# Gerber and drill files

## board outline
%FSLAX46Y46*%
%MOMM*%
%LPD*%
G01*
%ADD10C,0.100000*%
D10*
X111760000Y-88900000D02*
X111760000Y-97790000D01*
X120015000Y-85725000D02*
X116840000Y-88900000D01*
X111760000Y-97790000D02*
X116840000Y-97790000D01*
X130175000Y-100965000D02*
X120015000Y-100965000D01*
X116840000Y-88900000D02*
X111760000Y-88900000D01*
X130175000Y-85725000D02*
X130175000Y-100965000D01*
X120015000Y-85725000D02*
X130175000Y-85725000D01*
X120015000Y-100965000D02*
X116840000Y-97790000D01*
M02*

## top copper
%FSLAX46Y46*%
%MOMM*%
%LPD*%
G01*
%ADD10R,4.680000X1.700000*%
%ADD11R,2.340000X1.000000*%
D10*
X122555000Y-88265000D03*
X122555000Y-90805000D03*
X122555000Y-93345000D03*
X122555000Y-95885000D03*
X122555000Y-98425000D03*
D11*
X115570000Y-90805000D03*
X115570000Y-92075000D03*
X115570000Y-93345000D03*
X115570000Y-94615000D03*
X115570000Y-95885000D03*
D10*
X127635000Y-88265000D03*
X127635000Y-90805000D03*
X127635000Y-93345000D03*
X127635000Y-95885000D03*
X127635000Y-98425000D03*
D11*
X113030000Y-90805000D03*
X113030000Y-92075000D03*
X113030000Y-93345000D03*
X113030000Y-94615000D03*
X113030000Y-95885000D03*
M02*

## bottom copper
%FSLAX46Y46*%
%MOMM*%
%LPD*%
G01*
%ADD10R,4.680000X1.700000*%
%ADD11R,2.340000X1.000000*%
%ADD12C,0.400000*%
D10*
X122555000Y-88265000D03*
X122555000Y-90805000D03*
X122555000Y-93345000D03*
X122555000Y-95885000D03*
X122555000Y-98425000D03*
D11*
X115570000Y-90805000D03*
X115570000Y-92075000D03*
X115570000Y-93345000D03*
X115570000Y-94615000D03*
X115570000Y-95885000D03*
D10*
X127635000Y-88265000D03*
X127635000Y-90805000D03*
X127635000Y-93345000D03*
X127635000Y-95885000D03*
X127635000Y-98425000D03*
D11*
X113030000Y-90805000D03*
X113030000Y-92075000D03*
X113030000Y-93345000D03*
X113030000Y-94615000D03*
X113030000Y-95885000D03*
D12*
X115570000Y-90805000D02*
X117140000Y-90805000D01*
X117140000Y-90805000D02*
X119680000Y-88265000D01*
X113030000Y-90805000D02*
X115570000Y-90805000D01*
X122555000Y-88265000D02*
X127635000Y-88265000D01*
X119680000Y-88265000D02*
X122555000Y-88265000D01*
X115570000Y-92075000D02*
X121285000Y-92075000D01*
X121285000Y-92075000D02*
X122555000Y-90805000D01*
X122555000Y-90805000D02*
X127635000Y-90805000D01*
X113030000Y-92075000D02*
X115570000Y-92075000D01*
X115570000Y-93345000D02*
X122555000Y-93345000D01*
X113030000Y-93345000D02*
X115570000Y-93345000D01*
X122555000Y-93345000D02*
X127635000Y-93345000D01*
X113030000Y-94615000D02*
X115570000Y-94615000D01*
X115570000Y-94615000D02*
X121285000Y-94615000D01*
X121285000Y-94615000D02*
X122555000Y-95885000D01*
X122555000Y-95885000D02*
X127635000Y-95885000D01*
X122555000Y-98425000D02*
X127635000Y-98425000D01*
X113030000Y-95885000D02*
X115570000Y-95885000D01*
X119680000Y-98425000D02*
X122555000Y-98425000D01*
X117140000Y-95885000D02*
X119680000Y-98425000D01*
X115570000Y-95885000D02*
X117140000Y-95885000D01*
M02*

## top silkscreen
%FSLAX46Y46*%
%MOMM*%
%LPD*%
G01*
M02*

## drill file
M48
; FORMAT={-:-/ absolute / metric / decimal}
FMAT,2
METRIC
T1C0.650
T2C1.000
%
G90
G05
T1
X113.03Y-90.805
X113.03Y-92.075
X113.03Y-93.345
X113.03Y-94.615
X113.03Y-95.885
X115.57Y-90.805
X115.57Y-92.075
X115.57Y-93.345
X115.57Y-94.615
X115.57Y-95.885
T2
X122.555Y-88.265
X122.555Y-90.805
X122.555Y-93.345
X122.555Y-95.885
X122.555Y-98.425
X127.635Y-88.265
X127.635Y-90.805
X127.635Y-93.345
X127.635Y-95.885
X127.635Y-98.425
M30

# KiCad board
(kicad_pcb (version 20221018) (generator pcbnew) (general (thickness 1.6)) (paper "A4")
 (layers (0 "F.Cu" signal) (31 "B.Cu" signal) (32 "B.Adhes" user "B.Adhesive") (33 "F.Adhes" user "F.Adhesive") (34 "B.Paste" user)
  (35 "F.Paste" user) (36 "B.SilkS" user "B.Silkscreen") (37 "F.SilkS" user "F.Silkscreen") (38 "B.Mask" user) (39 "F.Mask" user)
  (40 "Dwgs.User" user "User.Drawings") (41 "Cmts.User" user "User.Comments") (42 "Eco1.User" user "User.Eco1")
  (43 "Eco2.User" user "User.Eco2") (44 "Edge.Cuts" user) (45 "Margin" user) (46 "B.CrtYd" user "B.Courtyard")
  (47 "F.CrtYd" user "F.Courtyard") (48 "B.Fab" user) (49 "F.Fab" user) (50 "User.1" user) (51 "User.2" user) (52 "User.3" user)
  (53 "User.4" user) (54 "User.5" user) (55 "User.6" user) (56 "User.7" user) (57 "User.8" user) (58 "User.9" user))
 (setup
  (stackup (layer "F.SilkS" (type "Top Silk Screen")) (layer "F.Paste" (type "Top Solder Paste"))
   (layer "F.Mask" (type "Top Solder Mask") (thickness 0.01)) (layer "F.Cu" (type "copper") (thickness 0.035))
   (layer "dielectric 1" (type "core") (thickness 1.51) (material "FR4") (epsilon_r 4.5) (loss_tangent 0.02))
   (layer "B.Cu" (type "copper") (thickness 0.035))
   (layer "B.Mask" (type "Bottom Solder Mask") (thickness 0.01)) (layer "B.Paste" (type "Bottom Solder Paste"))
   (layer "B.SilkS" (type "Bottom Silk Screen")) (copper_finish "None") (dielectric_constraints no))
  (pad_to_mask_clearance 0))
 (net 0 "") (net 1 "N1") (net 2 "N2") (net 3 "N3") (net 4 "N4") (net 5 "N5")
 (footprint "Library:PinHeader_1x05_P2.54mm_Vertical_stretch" (layer "F.Cu") (at 122.555 88.265)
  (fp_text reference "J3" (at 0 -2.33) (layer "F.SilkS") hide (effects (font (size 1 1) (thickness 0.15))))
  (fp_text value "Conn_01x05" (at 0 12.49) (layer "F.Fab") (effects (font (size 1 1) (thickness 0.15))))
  (pad "1" thru_hole rect (at 0 0) (size 4.68 1.7) (drill 1) (layers "*.Cu" "*.Mask") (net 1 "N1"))
  (pad "2" thru_hole rect (at 0 2.54) (size 4.68 1.7) (drill 1) (layers "*.Cu" "*.Mask") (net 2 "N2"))
  (pad "3" thru_hole rect (at 0 5.08) (size 4.68 1.7) (drill 1) (layers "*.Cu" "*.Mask") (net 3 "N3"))
  (pad "4" thru_hole rect (at 0 7.62) (size 4.68 1.7) (drill 1) (layers "*.Cu" "*.Mask") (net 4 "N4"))
  (pad "5" thru_hole rect (at 0 10.16) (size 4.68 1.7) (drill 1) (layers "*.Cu" "*.Mask") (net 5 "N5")))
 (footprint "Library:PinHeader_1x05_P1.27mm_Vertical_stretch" (layer "F.Cu") (at 115.57 90.805)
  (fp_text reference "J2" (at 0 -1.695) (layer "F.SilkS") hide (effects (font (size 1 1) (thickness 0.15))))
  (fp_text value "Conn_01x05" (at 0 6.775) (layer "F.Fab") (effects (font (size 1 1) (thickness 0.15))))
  (pad "1" thru_hole rect (at 0 0) (size 2.34 1) (drill 0.65) (layers "*.Cu" "*.Mask") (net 1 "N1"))
  (pad "2" thru_hole rect (at 0 1.27) (size 2.34 1) (drill 0.65) (layers "*.Cu" "*.Mask") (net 2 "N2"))
  (pad "3" thru_hole rect (at 0 2.54) (size 2.34 1) (drill 0.65) (layers "*.Cu" "*.Mask") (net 3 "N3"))
  (pad "4" thru_hole rect (at 0 3.81) (size 2.34 1) (drill 0.65) (layers "*.Cu" "*.Mask") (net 4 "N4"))
  (pad "5" thru_hole rect (at 0 5.08) (size 2.34 1) (drill 0.65) (layers "*.Cu" "*.Mask") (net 5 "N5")))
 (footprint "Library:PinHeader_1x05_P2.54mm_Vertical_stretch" (layer "F.Cu") (at 127.635 88.265)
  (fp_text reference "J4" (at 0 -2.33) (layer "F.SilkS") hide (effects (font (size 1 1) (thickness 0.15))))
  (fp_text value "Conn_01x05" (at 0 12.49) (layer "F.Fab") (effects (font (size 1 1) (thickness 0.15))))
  (pad "1" thru_hole rect (at 0 0) (size 4.68 1.7) (drill 1) (layers "*.Cu" "*.Mask") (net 1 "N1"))
  (pad "2" thru_hole rect (at 0 2.54) (size 4.68 1.7) (drill 1) (layers "*.Cu" "*.Mask") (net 2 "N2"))
  (pad "3" thru_hole rect (at 0 5.08) (size 4.68 1.7) (drill 1) (layers "*.Cu" "*.Mask") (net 3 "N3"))
  (pad "4" thru_hole rect (at 0 7.62) (size 4.68 1.7) (drill 1) (layers "*.Cu" "*.Mask") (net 4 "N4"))
  (pad "5" thru_hole rect (at 0 10.16) (size 4.68 1.7) (drill 1) (layers "*.Cu" "*.Mask") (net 5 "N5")))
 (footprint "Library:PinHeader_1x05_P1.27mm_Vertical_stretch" (layer "F.Cu") (at 113.03 90.805)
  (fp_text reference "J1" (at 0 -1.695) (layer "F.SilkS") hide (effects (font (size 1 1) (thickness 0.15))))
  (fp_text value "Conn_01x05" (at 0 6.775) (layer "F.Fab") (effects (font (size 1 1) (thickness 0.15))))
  (pad "1" thru_hole rect (at 0 0) (size 2.34 1) (drill 0.65) (layers "*.Cu" "*.Mask") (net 1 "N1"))
  (pad "2" thru_hole rect (at 0 1.27) (size 2.34 1) (drill 0.65) (layers "*.Cu" "*.Mask") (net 2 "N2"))
  (pad "3" thru_hole rect (at 0 2.54) (size 2.34 1) (drill 0.65) (layers "*.Cu" "*.Mask") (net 3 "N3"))
  (pad "4" thru_hole rect (at 0 3.81) (size 2.34 1) (drill 0.65) (layers "*.Cu" "*.Mask") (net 4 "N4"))
  (pad "5" thru_hole rect (at 0 5.08) (size 2.34 1) (drill 0.65) (layers "*.Cu" "*.Mask") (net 5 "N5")))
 (gr_line (start 111.76 88.9) (end 111.76 97.79) (stroke (width 0.1) (type default)) (layer "Edge.Cuts"))
 (gr_line (start 120.015 85.725) (end 116.84 88.9) (stroke (width 0.1) (type default)) (layer "Edge.Cuts"))
 (gr_line (start 111.76 97.79) (end 116.84 97.79) (stroke (width 0.1) (type default)) (layer "Edge.Cuts"))
 (gr_line (start 130.175 100.965) (end 120.015 100.965) (stroke (width 0.1) (type default)) (layer "Edge.Cuts"))
 (gr_line (start 116.84 88.9) (end 111.76 88.9) (stroke (width 0.1) (type default)) (layer "Edge.Cuts"))
 (gr_line (start 130.175 85.725) (end 130.175 100.965) (stroke (width 0.1) (type default)) (layer "Edge.Cuts"))
 (gr_line (start 120.015 85.725) (end 130.175 85.725) (stroke (width 0.1) (type default)) (layer "Edge.Cuts"))
 (gr_line (start 120.015 100.965) (end 116.84 97.79) (stroke (width 0.1) (type default)) (layer "Edge.Cuts"))
 (segment (start 115.57 90.805) (end 117.14 90.805) (width 0.4) (layer "B.Cu") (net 1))
 (segment (start 117.14 90.805) (end 119.68 88.265) (width 0.4) (layer "B.Cu") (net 1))
 (segment (start 113.03 90.805) (end 115.57 90.805) (width 0.4) (layer "B.Cu") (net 1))
 (segment (start 122.555 88.265) (end 127.635 88.265) (width 0.4) (layer "B.Cu") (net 1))
 (segment (start 119.68 88.265) (end 122.555 88.265) (width 0.4) (layer "B.Cu") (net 1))
 (segment (start 115.57 92.075) (end 121.285 92.075) (width 0.4) (layer "B.Cu") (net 2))
 (segment (start 121.285 92.075) (end 122.555 90.805) (width 0.4) (layer "B.Cu") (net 2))
 (segment (start 122.555 90.805) (end 127.635 90.805) (width 0.4) (layer "B.Cu") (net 2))
 (segment (start 113.03 92.075) (end 115.57 92.075) (width 0.4) (layer "B.Cu") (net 2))
 (segment (start 115.57 93.345) (end 122.555 93.345) (width 0.4) (layer "B.Cu") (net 3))
 (segment (start 113.03 93.345) (end 115.57 93.345) (width 0.4) (layer "B.Cu") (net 3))
 (segment (start 122.555 93.345) (end 127.635 93.345) (width 0.4) (layer "B.Cu") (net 3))
 (segment (start 113.03 94.615) (end 115.57 94.615) (width 0.4) (layer "B.Cu") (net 4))
 (segment (start 115.57 94.615) (end 121.285 94.615) (width 0.4) (layer "B.Cu") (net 4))
 (segment (start 121.285 94.615) (end 122.555 95.885) (width 0.4) (layer "B.Cu") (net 4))
 (segment (start 122.555 95.885) (end 127.635 95.885) (width 0.4) (layer "B.Cu") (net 4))
 (segment (start 122.555 98.425) (end 127.635 98.425) (width 0.4) (layer "B.Cu") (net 5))
 (segment (start 113.03 95.885) (end 115.57 95.885) (width 0.4) (layer "B.Cu") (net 5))
 (segment (start 119.68 98.425) (end 122.555 98.425) (width 0.4) (layer "B.Cu") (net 5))
 (segment (start 117.14 95.885) (end 119.68 98.425) (width 0.4) (layer "B.Cu") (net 5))
 (segment (start 115.57 95.885) (end 117.14 95.885) (width 0.4) (layer "B.Cu") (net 5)))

